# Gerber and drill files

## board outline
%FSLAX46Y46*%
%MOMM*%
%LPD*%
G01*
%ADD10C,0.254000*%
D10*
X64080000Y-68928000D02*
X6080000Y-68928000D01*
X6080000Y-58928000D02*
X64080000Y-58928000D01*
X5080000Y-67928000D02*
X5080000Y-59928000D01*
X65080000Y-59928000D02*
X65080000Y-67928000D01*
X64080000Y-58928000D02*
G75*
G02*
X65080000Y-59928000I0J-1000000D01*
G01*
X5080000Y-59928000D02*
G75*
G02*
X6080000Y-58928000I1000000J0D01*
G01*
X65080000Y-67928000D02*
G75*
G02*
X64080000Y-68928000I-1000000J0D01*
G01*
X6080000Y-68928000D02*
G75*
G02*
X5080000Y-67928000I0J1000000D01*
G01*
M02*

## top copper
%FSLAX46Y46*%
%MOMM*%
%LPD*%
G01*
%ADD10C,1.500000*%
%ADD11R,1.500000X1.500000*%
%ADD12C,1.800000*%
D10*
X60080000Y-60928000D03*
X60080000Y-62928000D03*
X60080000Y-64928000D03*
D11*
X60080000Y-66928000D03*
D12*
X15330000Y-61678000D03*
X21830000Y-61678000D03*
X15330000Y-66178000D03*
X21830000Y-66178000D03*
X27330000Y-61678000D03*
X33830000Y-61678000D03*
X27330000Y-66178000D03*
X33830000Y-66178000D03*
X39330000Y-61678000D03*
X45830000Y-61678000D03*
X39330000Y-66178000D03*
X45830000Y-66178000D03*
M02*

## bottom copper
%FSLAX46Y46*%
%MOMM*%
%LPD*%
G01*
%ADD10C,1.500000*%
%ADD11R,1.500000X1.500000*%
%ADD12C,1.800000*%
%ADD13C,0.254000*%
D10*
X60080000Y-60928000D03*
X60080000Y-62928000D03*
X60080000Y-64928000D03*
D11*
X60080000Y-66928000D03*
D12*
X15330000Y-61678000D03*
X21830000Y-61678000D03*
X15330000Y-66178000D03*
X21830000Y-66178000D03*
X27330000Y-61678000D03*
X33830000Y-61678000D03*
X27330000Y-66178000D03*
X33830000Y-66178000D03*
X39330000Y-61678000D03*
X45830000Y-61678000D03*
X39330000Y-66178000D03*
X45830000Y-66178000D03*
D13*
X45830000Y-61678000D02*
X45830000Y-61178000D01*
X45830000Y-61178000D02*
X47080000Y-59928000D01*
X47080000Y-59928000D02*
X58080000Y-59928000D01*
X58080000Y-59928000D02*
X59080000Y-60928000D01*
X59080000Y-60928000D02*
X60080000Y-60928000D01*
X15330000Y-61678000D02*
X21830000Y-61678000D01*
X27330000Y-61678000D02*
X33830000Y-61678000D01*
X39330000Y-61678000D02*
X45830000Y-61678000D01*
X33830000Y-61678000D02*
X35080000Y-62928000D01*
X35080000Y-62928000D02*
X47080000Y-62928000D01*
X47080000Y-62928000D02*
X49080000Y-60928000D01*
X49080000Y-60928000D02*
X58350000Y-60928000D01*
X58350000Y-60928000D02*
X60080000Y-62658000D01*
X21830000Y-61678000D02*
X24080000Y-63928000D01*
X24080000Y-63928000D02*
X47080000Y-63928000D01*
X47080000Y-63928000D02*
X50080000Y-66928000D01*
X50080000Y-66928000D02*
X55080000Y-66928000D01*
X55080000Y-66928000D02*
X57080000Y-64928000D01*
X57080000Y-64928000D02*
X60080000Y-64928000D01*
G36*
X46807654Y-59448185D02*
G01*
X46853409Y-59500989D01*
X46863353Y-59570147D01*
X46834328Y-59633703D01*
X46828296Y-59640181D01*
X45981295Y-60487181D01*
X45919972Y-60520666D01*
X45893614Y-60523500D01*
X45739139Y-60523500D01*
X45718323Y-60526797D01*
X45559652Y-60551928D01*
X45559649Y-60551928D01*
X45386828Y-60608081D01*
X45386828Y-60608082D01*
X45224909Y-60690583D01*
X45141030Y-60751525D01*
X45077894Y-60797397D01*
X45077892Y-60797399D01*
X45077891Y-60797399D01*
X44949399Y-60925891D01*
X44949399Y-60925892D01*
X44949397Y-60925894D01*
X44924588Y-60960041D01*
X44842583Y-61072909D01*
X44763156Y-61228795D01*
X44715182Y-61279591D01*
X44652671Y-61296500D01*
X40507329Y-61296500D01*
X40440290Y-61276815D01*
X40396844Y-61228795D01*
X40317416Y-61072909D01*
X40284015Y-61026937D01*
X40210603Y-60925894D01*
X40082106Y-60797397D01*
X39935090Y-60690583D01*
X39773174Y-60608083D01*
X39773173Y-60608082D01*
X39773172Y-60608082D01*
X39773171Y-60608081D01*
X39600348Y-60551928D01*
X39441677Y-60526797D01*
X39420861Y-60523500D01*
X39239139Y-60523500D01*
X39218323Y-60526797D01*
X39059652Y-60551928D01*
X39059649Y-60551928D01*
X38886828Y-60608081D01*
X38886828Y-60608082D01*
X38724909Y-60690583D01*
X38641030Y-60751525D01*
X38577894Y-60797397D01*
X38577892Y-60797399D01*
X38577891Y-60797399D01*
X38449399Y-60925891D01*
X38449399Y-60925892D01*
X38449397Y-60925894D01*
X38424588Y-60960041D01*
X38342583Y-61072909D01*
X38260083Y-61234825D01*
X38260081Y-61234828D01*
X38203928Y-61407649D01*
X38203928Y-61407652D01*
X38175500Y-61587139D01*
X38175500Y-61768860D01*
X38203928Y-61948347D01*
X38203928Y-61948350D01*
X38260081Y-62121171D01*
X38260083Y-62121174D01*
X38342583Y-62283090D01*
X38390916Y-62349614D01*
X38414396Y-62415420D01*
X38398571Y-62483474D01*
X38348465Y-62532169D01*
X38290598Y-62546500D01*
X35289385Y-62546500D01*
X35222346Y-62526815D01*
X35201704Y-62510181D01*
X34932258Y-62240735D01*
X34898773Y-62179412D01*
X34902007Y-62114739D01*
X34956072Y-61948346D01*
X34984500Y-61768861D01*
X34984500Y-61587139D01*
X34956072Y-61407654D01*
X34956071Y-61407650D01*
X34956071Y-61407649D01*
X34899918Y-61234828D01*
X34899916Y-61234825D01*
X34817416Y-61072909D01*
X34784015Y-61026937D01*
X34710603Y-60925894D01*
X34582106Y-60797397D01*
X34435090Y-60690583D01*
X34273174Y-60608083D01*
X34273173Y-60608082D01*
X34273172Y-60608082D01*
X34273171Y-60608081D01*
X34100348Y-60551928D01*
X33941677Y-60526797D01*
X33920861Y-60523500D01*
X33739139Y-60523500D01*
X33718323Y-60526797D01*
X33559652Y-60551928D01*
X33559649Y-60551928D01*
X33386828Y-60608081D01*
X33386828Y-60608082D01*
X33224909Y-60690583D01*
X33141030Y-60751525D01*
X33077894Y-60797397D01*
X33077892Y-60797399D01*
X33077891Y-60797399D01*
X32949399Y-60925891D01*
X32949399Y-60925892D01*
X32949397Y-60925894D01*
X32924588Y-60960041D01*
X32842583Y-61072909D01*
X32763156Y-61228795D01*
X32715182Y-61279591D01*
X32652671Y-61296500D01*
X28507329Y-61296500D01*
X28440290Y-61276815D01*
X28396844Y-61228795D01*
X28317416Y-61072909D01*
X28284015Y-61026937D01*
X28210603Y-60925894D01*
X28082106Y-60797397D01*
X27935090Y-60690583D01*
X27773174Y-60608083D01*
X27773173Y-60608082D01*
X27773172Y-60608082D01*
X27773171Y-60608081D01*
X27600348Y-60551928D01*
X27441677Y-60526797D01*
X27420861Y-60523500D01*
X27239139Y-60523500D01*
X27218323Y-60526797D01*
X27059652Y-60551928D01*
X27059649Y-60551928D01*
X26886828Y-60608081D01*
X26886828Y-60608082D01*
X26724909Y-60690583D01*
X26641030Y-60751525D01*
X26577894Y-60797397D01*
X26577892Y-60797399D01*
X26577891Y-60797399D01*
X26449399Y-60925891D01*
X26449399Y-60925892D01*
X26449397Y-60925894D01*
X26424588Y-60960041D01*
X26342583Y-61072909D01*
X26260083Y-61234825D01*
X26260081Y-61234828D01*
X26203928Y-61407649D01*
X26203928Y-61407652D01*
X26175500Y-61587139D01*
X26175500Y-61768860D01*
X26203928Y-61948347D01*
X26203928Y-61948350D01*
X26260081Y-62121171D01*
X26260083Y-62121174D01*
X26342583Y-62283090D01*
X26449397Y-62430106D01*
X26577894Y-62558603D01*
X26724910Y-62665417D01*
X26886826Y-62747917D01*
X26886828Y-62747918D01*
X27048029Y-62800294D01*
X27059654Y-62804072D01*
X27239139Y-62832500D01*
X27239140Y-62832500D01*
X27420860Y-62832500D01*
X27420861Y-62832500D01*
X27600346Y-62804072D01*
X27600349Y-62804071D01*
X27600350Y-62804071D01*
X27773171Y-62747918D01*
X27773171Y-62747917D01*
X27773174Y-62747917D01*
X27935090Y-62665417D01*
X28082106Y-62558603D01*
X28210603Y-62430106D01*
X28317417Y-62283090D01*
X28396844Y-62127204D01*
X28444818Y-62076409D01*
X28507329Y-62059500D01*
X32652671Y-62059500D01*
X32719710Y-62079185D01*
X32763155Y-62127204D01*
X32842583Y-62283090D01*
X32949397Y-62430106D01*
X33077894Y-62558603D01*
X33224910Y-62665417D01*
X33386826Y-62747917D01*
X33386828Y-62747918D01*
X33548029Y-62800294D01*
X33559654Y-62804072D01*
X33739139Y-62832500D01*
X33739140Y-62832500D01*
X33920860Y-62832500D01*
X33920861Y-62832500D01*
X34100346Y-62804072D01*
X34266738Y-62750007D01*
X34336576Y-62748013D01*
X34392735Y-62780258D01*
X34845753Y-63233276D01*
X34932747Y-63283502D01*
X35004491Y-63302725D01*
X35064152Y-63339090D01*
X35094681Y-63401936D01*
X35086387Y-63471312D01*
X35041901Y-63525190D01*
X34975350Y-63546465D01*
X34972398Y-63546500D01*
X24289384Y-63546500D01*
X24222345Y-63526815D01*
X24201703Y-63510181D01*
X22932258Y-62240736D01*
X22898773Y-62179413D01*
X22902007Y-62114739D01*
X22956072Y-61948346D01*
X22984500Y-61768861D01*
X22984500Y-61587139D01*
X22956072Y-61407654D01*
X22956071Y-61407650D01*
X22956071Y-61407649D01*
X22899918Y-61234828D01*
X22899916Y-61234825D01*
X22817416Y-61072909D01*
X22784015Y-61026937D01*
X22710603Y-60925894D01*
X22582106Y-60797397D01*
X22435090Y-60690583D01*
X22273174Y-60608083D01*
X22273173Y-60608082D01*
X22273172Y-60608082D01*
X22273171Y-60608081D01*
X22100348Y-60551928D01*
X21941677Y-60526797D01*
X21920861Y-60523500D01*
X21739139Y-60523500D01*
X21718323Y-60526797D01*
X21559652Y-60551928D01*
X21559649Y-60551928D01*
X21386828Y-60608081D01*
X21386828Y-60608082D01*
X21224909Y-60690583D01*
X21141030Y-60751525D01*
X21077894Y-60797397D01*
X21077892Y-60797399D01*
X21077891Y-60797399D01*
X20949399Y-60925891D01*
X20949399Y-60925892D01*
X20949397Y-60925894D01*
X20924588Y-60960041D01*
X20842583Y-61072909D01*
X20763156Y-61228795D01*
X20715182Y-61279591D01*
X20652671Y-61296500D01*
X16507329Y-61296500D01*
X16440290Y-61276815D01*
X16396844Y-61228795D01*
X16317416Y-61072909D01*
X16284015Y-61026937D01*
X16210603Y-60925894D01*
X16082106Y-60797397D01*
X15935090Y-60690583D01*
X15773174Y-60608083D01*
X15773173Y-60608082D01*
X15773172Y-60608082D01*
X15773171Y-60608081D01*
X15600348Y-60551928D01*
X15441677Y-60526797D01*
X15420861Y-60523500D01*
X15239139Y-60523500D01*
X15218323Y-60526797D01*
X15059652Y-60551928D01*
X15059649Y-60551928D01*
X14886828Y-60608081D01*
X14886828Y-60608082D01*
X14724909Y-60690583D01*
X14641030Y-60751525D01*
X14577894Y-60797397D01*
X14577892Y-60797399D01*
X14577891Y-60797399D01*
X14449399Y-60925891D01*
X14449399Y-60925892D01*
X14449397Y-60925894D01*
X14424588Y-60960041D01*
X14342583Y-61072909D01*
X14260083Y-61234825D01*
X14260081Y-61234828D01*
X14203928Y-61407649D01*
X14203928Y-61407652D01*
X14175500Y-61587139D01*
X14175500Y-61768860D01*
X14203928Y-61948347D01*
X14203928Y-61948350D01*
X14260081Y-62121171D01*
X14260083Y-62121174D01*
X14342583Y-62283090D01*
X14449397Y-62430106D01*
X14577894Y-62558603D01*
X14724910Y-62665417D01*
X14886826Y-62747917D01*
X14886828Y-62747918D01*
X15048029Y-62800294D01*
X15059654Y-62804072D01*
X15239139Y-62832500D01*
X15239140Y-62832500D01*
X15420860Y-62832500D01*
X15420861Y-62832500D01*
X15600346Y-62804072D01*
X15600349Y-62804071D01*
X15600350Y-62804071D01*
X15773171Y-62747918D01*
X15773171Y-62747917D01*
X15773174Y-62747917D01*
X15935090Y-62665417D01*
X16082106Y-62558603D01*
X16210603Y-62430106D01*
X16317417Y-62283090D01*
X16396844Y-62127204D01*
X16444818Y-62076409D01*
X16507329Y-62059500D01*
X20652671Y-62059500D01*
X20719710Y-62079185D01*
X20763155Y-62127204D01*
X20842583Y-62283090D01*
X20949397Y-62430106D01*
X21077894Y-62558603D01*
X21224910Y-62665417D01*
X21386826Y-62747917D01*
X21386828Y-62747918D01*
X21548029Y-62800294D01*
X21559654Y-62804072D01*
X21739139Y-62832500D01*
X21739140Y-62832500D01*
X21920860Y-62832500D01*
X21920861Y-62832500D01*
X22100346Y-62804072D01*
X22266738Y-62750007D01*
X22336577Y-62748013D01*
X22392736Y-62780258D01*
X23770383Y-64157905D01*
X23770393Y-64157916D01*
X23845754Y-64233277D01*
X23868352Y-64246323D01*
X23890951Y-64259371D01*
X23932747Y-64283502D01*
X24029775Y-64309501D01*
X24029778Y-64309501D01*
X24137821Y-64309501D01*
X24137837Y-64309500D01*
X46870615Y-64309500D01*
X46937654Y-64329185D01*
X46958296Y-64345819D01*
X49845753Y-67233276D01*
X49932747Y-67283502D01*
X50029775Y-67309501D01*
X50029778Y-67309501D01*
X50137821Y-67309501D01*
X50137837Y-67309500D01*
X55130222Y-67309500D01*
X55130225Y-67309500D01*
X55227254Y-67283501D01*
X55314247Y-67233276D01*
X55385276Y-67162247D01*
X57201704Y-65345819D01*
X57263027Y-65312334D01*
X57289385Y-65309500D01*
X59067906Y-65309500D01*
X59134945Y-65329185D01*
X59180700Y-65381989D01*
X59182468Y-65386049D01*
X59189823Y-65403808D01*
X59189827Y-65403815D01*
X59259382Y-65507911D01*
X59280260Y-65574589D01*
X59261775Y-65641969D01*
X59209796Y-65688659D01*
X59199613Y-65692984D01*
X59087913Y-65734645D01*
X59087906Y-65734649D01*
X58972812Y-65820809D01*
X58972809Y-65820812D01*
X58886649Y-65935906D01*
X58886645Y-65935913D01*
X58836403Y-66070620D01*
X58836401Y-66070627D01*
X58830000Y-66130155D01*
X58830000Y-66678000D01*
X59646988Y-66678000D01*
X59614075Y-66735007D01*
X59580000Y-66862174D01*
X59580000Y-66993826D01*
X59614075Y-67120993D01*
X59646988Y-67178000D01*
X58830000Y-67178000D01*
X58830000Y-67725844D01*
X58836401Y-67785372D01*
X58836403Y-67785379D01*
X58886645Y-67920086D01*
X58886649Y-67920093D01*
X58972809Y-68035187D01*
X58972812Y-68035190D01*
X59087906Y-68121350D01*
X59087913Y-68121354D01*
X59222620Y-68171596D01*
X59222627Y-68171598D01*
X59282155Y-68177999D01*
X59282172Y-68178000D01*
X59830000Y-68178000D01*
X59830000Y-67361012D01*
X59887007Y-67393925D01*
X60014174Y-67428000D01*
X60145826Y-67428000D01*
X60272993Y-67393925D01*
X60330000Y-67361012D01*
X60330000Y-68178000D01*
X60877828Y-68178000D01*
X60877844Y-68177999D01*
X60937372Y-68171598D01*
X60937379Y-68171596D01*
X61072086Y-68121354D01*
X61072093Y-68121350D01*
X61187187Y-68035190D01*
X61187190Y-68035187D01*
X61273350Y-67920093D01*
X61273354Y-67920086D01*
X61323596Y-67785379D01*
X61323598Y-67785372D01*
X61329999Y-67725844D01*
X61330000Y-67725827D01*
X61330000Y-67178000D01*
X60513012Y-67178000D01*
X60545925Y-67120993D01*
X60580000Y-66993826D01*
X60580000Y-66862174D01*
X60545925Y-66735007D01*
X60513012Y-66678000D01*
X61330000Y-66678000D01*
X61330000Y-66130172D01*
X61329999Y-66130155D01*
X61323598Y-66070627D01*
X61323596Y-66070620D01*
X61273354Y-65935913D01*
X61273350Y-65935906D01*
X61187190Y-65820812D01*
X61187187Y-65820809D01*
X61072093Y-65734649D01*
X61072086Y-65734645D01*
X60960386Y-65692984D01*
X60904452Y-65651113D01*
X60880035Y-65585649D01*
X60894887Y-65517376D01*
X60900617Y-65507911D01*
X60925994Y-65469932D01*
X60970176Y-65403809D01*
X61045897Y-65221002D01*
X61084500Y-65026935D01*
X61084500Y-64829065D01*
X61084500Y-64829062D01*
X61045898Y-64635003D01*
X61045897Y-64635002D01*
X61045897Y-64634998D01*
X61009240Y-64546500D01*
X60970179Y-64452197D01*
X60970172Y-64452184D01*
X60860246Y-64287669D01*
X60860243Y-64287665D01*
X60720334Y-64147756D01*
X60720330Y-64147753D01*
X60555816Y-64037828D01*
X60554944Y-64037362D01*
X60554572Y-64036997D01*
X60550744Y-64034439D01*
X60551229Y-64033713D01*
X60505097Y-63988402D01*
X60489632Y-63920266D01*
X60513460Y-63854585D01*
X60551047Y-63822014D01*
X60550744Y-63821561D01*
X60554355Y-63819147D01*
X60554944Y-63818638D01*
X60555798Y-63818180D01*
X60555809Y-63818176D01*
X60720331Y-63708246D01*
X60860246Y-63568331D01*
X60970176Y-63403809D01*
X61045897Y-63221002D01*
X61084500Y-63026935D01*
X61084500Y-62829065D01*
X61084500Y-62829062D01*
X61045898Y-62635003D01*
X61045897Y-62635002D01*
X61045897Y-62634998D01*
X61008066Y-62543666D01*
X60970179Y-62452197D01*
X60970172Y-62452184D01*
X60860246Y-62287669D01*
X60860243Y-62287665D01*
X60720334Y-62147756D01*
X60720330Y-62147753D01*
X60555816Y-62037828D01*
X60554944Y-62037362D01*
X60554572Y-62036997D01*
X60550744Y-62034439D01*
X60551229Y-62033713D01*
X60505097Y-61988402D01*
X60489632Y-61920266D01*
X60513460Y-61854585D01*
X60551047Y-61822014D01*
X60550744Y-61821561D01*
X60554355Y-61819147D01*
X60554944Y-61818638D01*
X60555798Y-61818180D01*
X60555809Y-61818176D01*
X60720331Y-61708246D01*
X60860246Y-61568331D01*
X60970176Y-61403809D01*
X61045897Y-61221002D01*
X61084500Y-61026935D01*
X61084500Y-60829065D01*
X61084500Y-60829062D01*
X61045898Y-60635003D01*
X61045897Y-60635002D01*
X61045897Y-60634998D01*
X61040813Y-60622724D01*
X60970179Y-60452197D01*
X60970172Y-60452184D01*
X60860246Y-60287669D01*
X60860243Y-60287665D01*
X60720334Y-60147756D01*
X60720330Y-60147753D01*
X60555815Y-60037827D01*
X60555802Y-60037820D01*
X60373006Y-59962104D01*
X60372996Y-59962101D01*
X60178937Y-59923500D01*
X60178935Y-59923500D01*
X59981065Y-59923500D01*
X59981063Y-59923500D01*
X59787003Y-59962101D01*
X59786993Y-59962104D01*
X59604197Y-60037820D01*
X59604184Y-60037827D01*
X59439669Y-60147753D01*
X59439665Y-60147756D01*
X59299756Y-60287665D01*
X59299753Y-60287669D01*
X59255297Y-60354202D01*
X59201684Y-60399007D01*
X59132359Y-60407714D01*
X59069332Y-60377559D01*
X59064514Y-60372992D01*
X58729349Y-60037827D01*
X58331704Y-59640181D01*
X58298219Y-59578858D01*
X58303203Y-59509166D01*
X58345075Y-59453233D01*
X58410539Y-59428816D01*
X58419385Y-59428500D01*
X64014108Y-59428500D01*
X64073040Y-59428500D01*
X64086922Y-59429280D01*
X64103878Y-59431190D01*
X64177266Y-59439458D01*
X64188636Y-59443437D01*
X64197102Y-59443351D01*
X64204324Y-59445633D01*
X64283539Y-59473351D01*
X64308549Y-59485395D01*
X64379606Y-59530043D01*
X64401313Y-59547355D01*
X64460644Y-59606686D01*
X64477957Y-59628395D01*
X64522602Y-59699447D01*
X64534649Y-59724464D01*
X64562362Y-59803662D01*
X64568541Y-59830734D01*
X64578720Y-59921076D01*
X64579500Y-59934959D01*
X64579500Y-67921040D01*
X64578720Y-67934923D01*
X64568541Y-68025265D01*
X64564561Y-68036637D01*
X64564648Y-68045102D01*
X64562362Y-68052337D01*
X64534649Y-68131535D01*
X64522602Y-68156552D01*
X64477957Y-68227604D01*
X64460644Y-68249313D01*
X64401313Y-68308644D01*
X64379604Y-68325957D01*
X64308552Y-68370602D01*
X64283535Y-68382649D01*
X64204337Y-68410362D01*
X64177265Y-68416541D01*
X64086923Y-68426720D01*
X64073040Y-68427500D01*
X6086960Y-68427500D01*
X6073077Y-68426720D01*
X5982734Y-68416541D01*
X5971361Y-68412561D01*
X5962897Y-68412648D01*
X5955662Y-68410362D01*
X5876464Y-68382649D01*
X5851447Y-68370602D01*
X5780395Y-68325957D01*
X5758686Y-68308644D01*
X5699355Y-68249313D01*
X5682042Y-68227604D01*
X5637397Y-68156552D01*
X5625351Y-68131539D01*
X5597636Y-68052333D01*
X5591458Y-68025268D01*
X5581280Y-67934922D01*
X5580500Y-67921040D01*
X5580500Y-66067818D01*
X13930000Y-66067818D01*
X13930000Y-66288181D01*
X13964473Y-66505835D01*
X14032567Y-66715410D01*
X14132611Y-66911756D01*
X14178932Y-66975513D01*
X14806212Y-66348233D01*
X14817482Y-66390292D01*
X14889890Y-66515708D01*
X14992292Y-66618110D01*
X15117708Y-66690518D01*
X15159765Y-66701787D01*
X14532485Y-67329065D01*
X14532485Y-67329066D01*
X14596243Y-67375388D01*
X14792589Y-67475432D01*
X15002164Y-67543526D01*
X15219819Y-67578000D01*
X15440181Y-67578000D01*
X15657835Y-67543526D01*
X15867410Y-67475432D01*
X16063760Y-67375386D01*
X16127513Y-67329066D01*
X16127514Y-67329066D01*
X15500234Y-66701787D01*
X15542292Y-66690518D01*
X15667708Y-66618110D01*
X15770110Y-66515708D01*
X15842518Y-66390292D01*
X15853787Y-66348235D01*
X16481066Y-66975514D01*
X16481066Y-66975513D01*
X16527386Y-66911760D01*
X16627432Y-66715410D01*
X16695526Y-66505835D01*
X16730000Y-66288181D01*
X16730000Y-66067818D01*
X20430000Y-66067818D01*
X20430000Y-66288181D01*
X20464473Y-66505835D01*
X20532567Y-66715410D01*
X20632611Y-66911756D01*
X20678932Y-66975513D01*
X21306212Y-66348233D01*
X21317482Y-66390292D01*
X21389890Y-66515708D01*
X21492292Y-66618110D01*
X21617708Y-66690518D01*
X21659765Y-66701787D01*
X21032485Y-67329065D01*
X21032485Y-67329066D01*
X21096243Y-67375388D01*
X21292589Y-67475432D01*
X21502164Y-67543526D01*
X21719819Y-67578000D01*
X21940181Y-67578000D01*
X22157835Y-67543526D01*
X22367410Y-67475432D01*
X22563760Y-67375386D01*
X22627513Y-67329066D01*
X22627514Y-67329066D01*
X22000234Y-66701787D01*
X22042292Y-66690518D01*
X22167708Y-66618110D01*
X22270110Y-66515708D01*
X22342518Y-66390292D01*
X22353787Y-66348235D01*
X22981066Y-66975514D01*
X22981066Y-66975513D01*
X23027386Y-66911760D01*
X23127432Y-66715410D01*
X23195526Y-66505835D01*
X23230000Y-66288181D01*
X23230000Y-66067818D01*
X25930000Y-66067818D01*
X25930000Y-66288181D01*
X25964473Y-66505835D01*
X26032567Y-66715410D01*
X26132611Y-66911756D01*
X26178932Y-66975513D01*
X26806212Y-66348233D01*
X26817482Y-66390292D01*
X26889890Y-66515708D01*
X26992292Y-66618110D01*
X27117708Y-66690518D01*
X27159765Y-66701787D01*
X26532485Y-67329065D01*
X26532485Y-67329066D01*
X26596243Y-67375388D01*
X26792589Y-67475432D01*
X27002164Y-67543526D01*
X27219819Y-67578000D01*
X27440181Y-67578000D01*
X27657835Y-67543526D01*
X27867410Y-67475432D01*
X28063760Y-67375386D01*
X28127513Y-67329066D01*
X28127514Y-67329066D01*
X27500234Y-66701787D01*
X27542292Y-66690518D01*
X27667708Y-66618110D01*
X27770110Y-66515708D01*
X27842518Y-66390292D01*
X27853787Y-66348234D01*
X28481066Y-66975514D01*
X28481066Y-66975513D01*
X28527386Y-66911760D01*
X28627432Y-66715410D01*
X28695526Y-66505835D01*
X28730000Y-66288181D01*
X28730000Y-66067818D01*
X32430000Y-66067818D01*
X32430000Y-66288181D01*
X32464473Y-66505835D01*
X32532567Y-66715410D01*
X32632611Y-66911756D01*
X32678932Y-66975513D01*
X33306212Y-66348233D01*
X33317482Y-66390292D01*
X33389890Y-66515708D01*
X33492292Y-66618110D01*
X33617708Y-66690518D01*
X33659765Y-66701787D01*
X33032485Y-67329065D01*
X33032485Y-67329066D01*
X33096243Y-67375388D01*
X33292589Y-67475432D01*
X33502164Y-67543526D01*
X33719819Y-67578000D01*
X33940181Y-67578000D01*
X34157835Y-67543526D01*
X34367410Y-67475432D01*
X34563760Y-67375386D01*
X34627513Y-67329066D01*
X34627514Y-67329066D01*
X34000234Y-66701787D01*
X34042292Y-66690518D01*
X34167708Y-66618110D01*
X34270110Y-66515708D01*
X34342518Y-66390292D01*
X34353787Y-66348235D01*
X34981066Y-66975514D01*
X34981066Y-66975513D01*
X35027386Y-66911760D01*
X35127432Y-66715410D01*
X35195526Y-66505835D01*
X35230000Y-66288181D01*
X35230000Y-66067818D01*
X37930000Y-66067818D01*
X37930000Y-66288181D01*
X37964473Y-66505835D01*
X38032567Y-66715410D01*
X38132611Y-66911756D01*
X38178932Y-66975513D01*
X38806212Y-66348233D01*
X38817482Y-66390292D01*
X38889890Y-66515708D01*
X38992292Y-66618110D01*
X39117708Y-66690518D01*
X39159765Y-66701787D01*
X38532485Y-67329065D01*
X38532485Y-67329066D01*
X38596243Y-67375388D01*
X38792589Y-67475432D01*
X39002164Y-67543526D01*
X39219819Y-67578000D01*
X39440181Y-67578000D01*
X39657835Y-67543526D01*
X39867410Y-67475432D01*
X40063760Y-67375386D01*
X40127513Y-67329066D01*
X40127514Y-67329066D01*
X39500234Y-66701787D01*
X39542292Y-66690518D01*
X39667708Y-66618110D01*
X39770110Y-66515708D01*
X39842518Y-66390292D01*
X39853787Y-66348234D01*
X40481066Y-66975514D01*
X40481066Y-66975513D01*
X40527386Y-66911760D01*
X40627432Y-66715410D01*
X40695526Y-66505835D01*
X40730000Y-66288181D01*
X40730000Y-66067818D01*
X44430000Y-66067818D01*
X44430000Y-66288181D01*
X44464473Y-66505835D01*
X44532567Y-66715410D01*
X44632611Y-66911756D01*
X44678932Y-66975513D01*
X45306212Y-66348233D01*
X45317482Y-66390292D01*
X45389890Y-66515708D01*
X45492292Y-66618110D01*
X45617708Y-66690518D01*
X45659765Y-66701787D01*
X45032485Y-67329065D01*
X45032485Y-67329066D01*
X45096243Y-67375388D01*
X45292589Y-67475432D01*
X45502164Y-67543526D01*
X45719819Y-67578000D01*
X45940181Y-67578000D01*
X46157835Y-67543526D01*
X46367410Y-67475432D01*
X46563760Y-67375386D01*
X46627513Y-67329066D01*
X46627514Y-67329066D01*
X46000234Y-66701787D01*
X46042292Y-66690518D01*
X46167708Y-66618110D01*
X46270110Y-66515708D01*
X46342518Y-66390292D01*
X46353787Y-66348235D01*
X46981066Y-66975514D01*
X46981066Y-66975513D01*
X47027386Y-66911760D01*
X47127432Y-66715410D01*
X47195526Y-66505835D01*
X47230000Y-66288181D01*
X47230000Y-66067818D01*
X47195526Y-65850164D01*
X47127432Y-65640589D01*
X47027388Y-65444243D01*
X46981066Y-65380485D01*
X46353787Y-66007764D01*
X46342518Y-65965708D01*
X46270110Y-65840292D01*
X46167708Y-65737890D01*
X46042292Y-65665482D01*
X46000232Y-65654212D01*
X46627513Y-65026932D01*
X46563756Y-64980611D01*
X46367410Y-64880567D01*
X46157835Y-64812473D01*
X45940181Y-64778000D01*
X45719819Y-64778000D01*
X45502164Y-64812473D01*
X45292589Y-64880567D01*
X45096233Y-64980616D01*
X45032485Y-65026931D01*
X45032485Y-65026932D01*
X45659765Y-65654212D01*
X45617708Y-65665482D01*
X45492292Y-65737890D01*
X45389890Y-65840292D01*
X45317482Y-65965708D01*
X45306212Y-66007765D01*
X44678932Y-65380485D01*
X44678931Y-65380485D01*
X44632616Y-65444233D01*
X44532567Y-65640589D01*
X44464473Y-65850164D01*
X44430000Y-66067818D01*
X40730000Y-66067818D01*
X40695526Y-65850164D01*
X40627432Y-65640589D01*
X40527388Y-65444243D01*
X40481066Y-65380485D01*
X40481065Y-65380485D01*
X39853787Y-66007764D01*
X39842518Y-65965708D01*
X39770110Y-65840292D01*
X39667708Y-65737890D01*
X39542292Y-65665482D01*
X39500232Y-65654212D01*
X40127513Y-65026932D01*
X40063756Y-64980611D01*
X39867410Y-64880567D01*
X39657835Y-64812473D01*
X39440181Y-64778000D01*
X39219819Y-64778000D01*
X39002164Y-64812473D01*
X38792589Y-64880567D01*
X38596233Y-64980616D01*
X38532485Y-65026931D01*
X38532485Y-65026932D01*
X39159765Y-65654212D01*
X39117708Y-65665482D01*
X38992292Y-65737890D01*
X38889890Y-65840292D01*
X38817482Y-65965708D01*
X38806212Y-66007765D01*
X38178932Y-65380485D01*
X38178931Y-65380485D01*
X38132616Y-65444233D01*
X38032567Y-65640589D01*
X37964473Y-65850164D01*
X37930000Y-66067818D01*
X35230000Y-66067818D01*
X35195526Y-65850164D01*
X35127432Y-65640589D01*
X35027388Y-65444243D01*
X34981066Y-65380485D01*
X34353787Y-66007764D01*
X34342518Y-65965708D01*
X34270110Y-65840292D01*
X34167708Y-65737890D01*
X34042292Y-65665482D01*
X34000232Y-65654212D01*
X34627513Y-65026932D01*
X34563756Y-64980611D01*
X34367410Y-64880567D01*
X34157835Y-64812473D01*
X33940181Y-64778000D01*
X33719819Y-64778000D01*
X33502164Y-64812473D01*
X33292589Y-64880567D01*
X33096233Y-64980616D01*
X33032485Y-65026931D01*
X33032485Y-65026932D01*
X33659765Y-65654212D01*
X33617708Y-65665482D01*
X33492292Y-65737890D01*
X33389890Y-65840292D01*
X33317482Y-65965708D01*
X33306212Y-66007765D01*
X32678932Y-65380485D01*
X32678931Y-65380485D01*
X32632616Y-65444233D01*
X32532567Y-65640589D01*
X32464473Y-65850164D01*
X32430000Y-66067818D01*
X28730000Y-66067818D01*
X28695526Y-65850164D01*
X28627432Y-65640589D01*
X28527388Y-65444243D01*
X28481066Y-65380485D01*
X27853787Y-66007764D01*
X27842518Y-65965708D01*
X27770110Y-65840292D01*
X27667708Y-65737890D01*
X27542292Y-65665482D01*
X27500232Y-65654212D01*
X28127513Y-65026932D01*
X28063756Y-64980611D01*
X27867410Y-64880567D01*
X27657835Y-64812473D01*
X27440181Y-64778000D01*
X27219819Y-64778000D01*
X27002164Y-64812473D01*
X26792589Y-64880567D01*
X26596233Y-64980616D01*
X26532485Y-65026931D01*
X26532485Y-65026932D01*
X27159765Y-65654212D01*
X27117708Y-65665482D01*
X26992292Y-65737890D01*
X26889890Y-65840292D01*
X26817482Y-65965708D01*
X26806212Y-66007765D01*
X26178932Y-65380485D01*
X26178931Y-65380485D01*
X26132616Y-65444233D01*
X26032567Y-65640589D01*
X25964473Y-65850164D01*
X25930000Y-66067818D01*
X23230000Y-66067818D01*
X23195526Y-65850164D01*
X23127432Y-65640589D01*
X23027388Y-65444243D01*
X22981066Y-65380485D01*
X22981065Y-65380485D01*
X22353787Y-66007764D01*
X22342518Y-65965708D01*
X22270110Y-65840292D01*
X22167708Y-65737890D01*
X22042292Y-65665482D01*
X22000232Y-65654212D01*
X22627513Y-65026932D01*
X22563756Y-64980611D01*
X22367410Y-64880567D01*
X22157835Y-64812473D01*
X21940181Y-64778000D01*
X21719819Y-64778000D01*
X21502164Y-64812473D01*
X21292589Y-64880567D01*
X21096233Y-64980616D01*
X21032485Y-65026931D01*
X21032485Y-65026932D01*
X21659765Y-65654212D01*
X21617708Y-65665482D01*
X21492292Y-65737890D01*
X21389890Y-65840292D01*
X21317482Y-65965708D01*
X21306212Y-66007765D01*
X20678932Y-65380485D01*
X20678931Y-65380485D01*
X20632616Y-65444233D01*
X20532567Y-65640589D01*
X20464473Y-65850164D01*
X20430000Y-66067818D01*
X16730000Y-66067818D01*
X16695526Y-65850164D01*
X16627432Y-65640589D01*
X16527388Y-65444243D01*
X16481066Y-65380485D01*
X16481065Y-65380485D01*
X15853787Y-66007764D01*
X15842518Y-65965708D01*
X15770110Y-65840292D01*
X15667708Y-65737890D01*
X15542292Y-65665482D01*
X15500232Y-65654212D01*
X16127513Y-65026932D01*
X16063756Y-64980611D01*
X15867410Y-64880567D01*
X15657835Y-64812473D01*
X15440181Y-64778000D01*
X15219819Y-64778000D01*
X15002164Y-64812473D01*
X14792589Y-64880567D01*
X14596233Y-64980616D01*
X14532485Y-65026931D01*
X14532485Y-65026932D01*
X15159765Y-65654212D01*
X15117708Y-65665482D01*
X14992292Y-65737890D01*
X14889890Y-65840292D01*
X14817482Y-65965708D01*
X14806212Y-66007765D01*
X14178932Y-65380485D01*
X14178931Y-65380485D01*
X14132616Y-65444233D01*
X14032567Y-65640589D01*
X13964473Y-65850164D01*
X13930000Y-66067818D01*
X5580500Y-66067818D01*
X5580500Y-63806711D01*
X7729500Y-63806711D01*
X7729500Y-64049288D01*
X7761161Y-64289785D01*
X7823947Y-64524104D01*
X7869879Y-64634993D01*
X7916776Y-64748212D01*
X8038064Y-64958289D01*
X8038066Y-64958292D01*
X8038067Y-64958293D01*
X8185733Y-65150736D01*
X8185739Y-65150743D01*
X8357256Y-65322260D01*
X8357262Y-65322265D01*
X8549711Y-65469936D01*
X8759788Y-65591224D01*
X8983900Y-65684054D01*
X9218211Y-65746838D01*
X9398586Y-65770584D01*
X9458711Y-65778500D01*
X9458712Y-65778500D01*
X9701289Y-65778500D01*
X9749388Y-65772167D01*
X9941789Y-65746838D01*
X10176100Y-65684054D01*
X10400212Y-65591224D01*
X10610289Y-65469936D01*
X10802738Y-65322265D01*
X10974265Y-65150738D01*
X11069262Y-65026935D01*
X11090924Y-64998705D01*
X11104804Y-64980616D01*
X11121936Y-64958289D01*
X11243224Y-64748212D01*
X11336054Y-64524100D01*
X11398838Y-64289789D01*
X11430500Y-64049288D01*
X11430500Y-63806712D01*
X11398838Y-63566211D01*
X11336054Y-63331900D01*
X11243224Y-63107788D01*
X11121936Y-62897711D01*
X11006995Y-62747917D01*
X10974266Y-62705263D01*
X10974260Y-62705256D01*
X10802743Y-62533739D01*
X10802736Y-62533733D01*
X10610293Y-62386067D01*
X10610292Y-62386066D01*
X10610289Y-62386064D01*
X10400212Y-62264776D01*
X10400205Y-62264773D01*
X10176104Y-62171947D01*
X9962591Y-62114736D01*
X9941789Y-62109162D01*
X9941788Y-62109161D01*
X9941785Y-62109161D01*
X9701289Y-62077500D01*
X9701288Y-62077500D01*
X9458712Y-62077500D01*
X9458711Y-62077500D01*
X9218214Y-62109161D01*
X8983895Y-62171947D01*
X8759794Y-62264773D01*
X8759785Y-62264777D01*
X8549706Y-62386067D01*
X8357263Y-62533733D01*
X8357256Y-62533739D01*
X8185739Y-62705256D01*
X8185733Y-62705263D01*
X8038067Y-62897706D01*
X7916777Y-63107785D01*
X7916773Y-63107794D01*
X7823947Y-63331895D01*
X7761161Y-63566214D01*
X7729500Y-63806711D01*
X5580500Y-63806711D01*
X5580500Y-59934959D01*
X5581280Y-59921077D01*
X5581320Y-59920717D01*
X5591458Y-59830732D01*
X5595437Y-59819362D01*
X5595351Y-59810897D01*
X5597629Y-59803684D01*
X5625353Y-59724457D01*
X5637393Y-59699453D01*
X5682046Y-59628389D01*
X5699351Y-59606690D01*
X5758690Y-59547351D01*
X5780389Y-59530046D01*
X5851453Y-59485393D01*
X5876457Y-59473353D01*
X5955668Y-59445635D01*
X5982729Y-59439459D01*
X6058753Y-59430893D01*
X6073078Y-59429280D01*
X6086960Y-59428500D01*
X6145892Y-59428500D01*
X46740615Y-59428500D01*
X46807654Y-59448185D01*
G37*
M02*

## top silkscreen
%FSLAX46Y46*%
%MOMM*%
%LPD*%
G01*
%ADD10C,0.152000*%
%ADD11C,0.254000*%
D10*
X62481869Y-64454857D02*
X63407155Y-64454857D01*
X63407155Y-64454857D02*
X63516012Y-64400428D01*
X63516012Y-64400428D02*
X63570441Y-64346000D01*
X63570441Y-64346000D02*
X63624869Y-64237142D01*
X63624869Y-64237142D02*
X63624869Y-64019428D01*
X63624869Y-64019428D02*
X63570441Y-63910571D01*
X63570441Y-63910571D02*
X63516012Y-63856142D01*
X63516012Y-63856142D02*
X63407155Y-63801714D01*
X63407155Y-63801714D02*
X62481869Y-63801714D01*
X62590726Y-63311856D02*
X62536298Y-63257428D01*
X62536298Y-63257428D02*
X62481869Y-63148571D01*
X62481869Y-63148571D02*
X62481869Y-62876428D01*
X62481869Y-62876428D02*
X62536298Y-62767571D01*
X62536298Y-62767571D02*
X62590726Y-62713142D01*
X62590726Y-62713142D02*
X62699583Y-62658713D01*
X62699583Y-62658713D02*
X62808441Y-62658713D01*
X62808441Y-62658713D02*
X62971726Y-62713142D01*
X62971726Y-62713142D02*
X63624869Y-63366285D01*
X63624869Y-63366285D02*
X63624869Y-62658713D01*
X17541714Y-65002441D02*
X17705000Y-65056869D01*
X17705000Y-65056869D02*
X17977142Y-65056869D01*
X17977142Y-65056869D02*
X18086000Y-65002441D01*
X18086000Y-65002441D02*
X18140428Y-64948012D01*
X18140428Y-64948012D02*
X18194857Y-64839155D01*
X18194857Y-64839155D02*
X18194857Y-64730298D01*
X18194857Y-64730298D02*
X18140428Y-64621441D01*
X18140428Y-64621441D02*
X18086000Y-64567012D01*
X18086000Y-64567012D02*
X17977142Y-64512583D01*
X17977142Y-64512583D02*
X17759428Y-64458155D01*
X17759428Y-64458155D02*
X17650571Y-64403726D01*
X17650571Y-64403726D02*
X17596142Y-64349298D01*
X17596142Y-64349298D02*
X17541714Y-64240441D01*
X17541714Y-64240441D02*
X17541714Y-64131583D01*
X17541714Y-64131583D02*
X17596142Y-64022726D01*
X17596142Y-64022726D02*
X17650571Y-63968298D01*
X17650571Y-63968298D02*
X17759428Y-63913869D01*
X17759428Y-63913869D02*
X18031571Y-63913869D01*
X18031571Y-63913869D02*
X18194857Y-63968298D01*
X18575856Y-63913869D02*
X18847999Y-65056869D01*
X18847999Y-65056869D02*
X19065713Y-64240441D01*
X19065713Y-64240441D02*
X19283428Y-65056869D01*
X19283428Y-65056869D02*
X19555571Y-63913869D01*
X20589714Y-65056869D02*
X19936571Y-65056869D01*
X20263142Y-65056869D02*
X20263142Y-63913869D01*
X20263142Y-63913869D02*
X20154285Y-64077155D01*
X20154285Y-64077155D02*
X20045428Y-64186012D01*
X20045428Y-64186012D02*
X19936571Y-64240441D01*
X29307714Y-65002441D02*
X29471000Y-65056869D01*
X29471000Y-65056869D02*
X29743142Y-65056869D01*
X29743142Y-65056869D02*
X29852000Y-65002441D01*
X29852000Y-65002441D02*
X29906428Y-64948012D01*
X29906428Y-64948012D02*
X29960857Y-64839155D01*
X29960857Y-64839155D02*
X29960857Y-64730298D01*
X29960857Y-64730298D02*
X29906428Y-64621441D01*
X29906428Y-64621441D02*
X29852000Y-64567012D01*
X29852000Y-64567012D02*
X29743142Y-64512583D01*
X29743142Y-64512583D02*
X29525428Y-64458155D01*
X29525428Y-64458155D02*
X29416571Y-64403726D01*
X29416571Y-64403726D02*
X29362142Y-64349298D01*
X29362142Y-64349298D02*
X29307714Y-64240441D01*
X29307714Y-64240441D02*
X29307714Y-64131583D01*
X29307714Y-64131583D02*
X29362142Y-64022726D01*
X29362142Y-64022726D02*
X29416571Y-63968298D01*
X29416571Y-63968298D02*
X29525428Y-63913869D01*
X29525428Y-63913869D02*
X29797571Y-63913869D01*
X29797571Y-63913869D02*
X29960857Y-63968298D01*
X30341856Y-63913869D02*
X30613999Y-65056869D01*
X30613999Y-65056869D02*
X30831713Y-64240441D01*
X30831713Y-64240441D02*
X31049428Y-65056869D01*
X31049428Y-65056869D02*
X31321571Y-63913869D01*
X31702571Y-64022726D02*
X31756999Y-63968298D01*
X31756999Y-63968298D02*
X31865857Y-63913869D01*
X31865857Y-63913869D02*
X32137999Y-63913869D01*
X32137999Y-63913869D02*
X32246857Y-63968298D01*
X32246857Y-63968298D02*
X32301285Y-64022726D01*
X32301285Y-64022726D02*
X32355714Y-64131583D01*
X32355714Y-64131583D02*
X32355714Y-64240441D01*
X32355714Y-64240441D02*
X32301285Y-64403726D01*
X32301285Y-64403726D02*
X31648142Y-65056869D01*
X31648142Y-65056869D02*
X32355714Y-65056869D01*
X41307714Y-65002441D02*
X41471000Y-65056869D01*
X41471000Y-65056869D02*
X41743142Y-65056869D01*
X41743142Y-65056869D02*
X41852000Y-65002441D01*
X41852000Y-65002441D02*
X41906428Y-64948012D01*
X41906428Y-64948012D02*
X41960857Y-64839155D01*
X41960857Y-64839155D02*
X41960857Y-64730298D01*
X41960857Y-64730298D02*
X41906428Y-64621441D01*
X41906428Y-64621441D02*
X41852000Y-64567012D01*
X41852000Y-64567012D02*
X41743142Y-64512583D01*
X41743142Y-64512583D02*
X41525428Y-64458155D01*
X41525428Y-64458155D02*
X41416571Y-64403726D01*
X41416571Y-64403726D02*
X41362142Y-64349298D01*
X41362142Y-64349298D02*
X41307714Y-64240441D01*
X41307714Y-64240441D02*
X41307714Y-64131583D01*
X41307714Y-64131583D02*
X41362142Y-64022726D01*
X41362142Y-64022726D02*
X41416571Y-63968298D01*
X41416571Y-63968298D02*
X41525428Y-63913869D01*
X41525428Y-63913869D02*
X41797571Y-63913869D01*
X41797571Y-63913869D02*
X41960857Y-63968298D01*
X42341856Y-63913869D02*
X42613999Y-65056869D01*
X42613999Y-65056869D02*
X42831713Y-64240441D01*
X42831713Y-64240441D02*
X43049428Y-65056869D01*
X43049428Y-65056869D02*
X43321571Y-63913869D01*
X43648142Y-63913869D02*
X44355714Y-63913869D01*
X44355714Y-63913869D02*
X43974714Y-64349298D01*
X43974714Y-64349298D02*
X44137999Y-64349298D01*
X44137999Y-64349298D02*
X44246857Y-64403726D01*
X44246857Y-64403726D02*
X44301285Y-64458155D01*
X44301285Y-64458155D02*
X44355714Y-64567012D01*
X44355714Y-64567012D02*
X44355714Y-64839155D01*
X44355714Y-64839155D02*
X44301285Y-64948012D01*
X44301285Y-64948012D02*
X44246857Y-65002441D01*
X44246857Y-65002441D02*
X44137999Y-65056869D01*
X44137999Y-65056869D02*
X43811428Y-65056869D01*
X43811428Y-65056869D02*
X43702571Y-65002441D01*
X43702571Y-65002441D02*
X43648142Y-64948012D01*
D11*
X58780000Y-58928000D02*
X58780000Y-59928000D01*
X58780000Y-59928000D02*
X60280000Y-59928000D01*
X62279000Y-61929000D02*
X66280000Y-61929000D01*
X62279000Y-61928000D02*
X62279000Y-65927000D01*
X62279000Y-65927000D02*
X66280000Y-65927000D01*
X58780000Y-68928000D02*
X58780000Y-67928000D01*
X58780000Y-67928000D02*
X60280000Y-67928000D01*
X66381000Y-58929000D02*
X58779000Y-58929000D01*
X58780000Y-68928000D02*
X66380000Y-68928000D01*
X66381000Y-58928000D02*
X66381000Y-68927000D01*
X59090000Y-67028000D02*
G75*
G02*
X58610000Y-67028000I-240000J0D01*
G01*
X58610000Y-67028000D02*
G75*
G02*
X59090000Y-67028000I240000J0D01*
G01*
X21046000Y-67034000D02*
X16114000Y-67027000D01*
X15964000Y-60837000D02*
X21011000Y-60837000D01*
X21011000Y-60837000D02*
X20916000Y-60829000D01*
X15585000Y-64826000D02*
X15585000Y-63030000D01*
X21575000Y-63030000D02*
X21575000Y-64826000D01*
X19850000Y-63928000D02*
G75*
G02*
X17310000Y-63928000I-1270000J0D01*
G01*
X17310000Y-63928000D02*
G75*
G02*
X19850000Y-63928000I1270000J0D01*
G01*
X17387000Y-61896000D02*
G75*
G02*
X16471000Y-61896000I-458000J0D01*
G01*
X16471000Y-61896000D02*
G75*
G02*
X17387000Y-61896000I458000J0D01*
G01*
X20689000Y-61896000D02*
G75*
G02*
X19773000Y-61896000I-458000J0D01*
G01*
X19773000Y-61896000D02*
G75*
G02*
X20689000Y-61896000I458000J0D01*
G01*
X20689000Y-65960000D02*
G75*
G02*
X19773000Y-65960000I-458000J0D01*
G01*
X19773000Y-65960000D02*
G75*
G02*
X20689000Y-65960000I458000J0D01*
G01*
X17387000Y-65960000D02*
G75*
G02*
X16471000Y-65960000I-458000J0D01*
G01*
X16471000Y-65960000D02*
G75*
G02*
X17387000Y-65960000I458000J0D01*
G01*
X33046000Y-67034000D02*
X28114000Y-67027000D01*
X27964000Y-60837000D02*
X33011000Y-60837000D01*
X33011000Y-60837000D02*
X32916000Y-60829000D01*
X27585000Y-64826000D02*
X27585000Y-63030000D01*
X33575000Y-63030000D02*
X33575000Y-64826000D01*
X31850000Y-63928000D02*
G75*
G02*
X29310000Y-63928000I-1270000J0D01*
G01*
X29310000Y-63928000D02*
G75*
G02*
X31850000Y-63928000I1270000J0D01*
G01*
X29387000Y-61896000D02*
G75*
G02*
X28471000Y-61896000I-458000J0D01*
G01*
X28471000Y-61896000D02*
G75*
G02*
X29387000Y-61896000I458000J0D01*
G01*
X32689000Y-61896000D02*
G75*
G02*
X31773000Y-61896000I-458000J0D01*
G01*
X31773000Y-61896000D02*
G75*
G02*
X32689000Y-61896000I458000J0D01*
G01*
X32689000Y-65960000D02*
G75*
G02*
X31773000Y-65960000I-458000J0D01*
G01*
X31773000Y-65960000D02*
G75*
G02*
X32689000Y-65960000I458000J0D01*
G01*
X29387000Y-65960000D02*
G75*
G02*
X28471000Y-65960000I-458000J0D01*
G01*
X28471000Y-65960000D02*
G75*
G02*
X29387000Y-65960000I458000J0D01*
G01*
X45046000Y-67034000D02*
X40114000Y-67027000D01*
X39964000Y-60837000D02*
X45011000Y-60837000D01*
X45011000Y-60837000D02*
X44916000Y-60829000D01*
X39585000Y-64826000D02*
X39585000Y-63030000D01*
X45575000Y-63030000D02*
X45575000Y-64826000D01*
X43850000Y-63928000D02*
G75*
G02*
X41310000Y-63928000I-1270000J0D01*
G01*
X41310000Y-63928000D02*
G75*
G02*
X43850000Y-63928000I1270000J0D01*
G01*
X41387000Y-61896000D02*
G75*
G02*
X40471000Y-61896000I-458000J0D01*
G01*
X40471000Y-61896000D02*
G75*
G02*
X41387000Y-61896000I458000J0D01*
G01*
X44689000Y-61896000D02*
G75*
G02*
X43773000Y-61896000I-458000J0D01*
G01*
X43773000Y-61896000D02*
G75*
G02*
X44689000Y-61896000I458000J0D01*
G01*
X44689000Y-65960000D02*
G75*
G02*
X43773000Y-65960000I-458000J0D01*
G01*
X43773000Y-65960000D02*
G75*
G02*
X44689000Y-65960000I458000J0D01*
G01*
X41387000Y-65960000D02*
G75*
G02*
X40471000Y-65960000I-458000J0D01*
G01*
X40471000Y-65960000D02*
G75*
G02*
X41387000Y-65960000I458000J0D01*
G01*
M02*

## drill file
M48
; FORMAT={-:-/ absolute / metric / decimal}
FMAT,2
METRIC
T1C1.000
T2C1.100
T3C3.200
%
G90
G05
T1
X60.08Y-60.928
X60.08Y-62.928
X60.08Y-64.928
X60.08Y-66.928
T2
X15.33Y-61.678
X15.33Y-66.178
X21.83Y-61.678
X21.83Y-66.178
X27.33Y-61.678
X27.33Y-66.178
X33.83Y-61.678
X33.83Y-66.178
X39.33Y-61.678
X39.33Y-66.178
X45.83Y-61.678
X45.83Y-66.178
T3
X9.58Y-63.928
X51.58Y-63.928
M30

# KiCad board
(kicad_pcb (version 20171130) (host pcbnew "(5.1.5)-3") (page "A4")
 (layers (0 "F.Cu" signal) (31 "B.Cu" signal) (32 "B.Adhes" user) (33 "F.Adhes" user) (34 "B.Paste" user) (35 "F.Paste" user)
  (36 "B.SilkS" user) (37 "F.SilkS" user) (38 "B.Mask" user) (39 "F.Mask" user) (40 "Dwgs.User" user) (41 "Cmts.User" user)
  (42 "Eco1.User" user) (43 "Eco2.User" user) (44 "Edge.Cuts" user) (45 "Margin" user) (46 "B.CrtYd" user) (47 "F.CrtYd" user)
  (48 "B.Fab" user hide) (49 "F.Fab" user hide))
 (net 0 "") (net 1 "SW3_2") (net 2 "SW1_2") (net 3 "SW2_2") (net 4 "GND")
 (gr_line (start 64.08 68.928) (end 6.08 68.928) (width 0.254) (layer "Edge.Cuts"))
 (gr_line (start 6.08 58.928) (end 64.08 58.928) (width 0.254) (layer "Edge.Cuts"))
 (gr_line (start 5.08 67.928) (end 5.08 59.928) (width 0.254) (layer "Edge.Cuts"))
 (gr_line (start 65.08 59.928) (end 65.08 67.928) (width 0.254) (layer "Edge.Cuts"))
 (gr_arc (start 64.08 59.928) (end 64.08 58.928) (angle 90) (width 0.254) (layer "Edge.Cuts"))
 (gr_arc (start 6.08 59.928) (end 5.08 59.928) (angle 90) (width 0.254) (layer "Edge.Cuts"))
 (gr_arc (start 64.08 67.928) (end 65.08 67.928) (angle 90) (width 0.254) (layer "Edge.Cuts"))
 (gr_arc (start 6.08 67.928) (end 6.08 68.928) (angle 90) (width 0.254) (layer "Edge.Cuts"))
 (segment (start 45.83 61.678) (end 45.83 61.178) (width 0.254) (layer "B.Cu") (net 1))
 (segment (start 45.83 61.178) (end 47.08 59.928) (width 0.254) (layer "B.Cu") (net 1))
 (segment (start 47.08 59.928) (end 58.08 59.928) (width 0.254) (layer "B.Cu") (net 1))
 (segment (start 58.08 59.928) (end 59.08 60.928) (width 0.254) (layer "B.Cu") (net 1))
 (segment (start 59.08 60.928) (end 60.08 60.928) (width 0.254) (layer "B.Cu") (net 1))
 (segment (start 15.33 61.678) (end 21.83 61.678) (width 0.254) (layer "B.Cu") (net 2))
 (segment (start 27.33 61.678) (end 33.83 61.678) (width 0.254) (layer "B.Cu") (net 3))
 (segment (start 39.33 61.678) (end 45.83 61.678) (width 0.254) (layer "B.Cu") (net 1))
 (segment (start 33.83 61.678) (end 35.08 62.928) (width 0.254) (layer "B.Cu") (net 3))
 (segment (start 35.08 62.928) (end 47.08 62.928) (width 0.254) (layer "B.Cu") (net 3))
 (segment (start 47.08 62.928) (end 49.08 60.928) (width 0.254) (layer "B.Cu") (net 3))
 (segment (start 49.08 60.928) (end 58.35 60.928) (width 0.254) (layer "B.Cu") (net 3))
 (segment (start 58.35 60.928) (end 60.08 62.658) (width 0.254) (layer "B.Cu") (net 3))
 (segment (start 21.83 61.678) (end 24.08 63.928) (width 0.254) (layer "B.Cu") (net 2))
 (segment (start 24.08 63.928) (end 47.08 63.928) (width 0.254) (layer "B.Cu") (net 2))
 (segment (start 47.08 63.928) (end 50.08 66.928) (width 0.254) (layer "B.Cu") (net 2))
 (segment (start 50.08 66.928) (end 55.08 66.928) (width 0.254) (layer "B.Cu") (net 2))
 (segment (start 55.08 66.928) (end 57.08 64.928) (width 0.254) (layer "B.Cu") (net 2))
 (segment (start 57.08 64.928) (end 60.08 64.928) (width 0.254) (layer "B.Cu") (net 2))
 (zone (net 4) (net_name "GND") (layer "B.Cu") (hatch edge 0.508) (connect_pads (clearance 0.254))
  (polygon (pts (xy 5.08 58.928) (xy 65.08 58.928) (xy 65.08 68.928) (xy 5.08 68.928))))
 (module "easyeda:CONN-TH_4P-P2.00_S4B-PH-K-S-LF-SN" (layer "F.Cu") (at 60.08 63.928 90)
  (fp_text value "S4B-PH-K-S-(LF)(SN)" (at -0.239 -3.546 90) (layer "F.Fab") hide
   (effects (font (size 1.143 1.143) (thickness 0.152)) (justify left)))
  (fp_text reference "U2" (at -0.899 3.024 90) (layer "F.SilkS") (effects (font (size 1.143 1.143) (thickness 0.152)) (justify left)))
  (fp_line (start 5 -1.3) (end 4 -1.3) (width 0.254) (layer "F.SilkS"))
  (fp_line (start 4 -1.3) (end 4 0.2) (width 0.254) (layer "F.SilkS"))
  (fp_line (start 1.999 2.199) (end 1.999 6.2) (width 0.254) (layer "F.SilkS"))
  (fp_line (start 2 2.199) (end -1.999 2.199) (width 0.254) (layer "F.SilkS"))
  (fp_line (start -1.999 2.199) (end -1.999 6.2) (width 0.254) (layer "F.SilkS"))
  (fp_line (start -5 -1.3) (end -4 -1.3) (width 0.254) (layer "F.SilkS"))
  (fp_line (start -4 -1.3) (end -4 0.2) (width 0.254) (layer "F.SilkS"))
  (fp_line (start 4.999 6.301) (end 4.999 -1.301) (width 0.254) (layer "F.SilkS"))
  (fp_line (start -5 -1.3) (end -5 6.3) (width 0.254) (layer "F.SilkS"))
  (fp_line (start 5 6.301) (end -4.999 6.301) (width 0.254) (layer "F.SilkS"))
  (fp_circle (center -3.1 -1.23) (end -2.86 -1.23) (layer "F.SilkS") (width 0.254))
  (pad 4 thru_hole circle (at 3 0 90) (size 1.5 1.5) (layers "*.Cu" "*.Paste" "*.Mask") (drill 1) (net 1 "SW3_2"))
  (pad 3 thru_hole circle (at 1 0 90) (size 1.5 1.5) (layers "*.Cu" "*.Paste" "*.Mask") (drill 1) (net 3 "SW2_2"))
  (pad 2 thru_hole circle (at -1 0 90) (size 1.5 1.5) (layers "*.Cu" "*.Paste" "*.Mask") (drill 1) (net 2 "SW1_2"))
  (pad 1 thru_hole rect (at -3 0 90) (size 1.5 1.5) (layers "*.Cu" "*.Paste" "*.Mask") (drill 1) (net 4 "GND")))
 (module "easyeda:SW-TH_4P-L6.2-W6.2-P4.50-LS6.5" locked (layer "F.Cu") (at 18.58 63.928)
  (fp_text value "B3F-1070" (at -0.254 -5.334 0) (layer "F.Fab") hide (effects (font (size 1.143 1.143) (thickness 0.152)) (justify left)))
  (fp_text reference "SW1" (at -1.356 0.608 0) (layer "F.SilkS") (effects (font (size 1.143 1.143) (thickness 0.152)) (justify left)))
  (fp_line (start 2.466 3.106) (end -2.466 3.099) (width 0.254) (layer "F.SilkS"))
  (fp_line (start -2.616 -3.091) (end 2.431 -3.091) (width 0.254) (layer "F.SilkS"))
  (fp_line (start 2.431 -3.091) (end 2.336 -3.099) (width 0.254) (layer "F.SilkS"))
  (fp_line (start -2.995 0.898) (end -2.995 -0.898) (width 0.254) (layer "F.SilkS"))
  (fp_line (start 2.995 -0.898) (end 2.995 0.898) (width 0.254) (layer "F.SilkS"))
  (fp_circle (center 0 0) (end 1.27 0) (layer "F.SilkS") (width 0.254))
  (fp_circle (center -1.651 -2.032) (end -1.193 -2.032) (layer "F.SilkS") (width 0.254))
  (fp_circle (center 1.651 -2.032) (end 2.109 -2.032) (layer "F.SilkS") (width 0.254))
  (fp_circle (center 1.651 2.032) (end 2.109 2.032) (layer "F.SilkS") (width 0.254))
  (fp_circle (center -1.651 2.032) (end -1.193 2.032) (layer "F.SilkS") (width 0.254))
  (pad 1 thru_hole circle (at -3.25 -2.25 0) (size 1.8 1.8) (layers "*.Cu" "*.Paste" "*.Mask") (drill 1.1) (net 2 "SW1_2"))
  (pad 2 thru_hole circle (at 3.25 -2.25 0) (size 1.8 1.8) (layers "*.Cu" "*.Paste" "*.Mask") (drill 1.1) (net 2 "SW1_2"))
  (pad 3 thru_hole circle (at -3.25 2.25 0) (size 1.8 1.8) (layers "*.Cu" "*.Paste" "*.Mask") (drill 1.1) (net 4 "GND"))
  (pad 4 thru_hole circle (at 3.25 2.25 0) (size 1.8 1.8) (layers "*.Cu" "*.Paste" "*.Mask") (drill 1.1) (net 4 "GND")))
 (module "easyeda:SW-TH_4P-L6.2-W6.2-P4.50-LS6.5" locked (layer "F.Cu") (at 30.58 63.928)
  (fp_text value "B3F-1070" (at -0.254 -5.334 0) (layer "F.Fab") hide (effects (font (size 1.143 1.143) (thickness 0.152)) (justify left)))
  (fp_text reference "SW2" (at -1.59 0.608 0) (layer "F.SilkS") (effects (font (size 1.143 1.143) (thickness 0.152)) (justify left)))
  (fp_line (start 2.466 3.106) (end -2.466 3.099) (width 0.254) (layer "F.SilkS"))
  (fp_line (start -2.616 -3.091) (end 2.431 -3.091) (width 0.254) (layer "F.SilkS"))
  (fp_line (start 2.431 -3.091) (end 2.336 -3.099) (width 0.254) (layer "F.SilkS"))
  (fp_line (start -2.995 0.898) (end -2.995 -0.898) (width 0.254) (layer "F.SilkS"))
  (fp_line (start 2.995 -0.898) (end 2.995 0.898) (width 0.254) (layer "F.SilkS"))
  (fp_circle (center 0 0) (end 1.27 0) (layer "F.SilkS") (width 0.254))
  (fp_circle (center -1.651 -2.032) (end -1.193 -2.032) (layer "F.SilkS") (width 0.254))
  (fp_circle (center 1.651 -2.032) (end 2.109 -2.032) (layer "F.SilkS") (width 0.254))
  (fp_circle (center 1.651 2.032) (end 2.109 2.032) (layer "F.SilkS") (width 0.254))
  (fp_circle (center -1.651 2.032) (end -1.193 2.032) (layer "F.SilkS") (width 0.254))
  (pad 1 thru_hole circle (at -3.25 -2.25 0) (size 1.8 1.8) (layers "*.Cu" "*.Paste" "*.Mask") (drill 1.1) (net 3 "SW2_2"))
  (pad 2 thru_hole circle (at 3.25 -2.25 0) (size 1.8 1.8) (layers "*.Cu" "*.Paste" "*.Mask") (drill 1.1) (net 3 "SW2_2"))
  (pad 3 thru_hole circle (at -3.25 2.25 0) (size 1.8 1.8) (layers "*.Cu" "*.Paste" "*.Mask") (drill 1.1) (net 4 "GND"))
  (pad 4 thru_hole circle (at 3.25 2.25 0) (size 1.8 1.8) (layers "*.Cu" "*.Paste" "*.Mask") (drill 1.1) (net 4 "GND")))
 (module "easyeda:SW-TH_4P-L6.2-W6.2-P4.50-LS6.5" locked (layer "F.Cu") (at 42.58 63.928)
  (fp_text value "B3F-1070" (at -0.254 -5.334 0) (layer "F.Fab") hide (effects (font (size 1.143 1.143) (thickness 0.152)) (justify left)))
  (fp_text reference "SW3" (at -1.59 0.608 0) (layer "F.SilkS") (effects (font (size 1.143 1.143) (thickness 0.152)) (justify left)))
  (fp_line (start 2.466 3.106) (end -2.466 3.099) (width 0.254) (layer "F.SilkS"))
  (fp_line (start -2.616 -3.091) (end 2.431 -3.091) (width 0.254) (layer "F.SilkS"))
  (fp_line (start 2.431 -3.091) (end 2.336 -3.099) (width 0.254) (layer "F.SilkS"))
  (fp_line (start -2.995 0.898) (end -2.995 -0.898) (width 0.254) (layer "F.SilkS"))
  (fp_line (start 2.995 -0.898) (end 2.995 0.898) (width 0.254) (layer "F.SilkS"))
  (fp_circle (center 0 0) (end 1.27 0) (layer "F.SilkS") (width 0.254))
  (fp_circle (center -1.651 -2.032) (end -1.193 -2.032) (layer "F.SilkS") (width 0.254))
  (fp_circle (center 1.651 -2.032) (end 2.109 -2.032) (layer "F.SilkS") (width 0.254))
  (fp_circle (center 1.651 2.032) (end 2.109 2.032) (layer "F.SilkS") (width 0.254))
  (fp_circle (center -1.651 2.032) (end -1.193 2.032) (layer "F.SilkS") (width 0.254))
  (pad 1 thru_hole circle (at -3.25 -2.25 0) (size 1.8 1.8) (layers "*.Cu" "*.Paste" "*.Mask") (drill 1.1) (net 1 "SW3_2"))
  (pad 2 thru_hole circle (at 3.25 -2.25 0) (size 1.8 1.8) (layers "*.Cu" "*.Paste" "*.Mask") (drill 1.1) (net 1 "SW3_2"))
  (pad 3 thru_hole circle (at -3.25 2.25 0) (size 1.8 1.8) (layers "*.Cu" "*.Paste" "*.Mask") (drill 1.1) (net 4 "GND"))
  (pad 4 thru_hole circle (at 3.25 2.25 0) (size 1.8 1.8) (layers "*.Cu" "*.Paste" "*.Mask") (drill 1.1) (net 4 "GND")))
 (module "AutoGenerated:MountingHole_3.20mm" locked (layer "F.Cu") (at 9.58 63.928) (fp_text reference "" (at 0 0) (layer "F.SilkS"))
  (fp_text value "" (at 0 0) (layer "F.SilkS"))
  (pad "" np_thru_hole circle (at 0 0) (size 3.2 3.2) (drill 3.2) (layers "*.Cu" "*.Mask")))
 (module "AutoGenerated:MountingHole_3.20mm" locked (layer "F.Cu") (at 51.58 63.928) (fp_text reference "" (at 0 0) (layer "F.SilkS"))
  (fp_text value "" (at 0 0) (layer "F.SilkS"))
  (pad "" np_thru_hole circle (at 0 0) (size 3.2 3.2) (drill 3.2) (layers "*.Cu" "*.Mask"))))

